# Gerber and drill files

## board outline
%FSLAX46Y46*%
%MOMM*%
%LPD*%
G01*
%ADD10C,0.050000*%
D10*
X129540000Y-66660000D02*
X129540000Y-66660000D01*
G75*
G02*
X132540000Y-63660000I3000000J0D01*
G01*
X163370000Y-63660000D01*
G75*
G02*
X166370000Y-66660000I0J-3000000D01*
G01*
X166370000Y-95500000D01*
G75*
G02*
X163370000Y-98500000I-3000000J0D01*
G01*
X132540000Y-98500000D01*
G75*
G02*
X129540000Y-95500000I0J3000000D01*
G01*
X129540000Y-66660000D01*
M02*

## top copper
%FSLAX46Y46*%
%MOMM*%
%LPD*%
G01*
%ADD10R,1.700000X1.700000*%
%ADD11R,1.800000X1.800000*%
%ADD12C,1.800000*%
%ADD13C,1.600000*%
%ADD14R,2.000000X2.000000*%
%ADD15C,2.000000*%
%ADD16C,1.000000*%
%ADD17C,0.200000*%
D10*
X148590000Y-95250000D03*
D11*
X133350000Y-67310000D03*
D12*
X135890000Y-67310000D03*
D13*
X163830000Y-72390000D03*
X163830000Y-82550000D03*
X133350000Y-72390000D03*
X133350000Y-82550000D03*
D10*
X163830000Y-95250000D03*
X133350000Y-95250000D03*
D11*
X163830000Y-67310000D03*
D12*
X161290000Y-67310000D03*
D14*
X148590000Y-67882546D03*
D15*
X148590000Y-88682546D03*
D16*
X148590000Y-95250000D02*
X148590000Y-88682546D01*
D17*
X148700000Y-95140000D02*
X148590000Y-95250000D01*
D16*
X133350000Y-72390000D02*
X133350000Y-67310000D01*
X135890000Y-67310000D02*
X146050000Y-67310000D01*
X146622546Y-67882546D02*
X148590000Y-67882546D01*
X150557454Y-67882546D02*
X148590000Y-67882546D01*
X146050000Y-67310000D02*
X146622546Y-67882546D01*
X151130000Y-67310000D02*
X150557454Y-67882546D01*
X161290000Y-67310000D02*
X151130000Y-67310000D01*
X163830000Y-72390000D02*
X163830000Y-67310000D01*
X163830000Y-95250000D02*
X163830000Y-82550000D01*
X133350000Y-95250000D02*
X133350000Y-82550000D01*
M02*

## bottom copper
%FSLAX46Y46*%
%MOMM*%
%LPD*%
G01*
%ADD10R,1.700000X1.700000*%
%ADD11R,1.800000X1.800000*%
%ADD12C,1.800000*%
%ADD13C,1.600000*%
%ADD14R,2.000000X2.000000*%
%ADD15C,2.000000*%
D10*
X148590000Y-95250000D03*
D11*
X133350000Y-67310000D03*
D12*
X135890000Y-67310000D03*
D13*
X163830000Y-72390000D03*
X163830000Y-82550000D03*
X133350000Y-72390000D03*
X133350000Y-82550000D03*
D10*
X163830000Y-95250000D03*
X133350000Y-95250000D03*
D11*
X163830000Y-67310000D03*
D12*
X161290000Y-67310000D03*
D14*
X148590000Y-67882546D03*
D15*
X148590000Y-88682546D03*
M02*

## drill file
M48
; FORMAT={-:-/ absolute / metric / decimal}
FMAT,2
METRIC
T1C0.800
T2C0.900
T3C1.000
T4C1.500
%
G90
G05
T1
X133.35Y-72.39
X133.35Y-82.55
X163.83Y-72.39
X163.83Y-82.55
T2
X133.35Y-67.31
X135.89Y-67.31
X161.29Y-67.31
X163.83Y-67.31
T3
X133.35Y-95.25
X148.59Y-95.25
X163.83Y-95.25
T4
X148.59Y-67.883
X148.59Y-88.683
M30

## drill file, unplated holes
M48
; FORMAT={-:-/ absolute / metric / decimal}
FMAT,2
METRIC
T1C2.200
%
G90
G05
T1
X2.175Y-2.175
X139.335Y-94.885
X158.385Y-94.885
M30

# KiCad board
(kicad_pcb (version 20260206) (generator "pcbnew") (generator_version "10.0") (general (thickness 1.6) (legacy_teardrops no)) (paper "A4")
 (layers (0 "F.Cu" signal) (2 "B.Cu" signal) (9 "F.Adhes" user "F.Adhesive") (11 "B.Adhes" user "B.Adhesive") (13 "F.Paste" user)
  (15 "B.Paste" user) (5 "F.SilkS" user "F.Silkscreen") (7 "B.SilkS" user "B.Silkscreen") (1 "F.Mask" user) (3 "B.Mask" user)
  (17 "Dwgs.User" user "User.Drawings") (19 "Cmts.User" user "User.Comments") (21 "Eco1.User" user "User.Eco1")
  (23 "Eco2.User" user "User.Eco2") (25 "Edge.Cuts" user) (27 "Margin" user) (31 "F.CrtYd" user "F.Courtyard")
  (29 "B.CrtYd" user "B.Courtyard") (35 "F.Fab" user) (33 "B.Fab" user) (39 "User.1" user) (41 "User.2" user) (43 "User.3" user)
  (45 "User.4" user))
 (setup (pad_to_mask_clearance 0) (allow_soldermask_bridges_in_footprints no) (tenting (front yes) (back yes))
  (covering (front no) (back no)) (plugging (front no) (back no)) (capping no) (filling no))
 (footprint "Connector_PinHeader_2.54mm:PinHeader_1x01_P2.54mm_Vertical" (layer "F.Cu") (at 148.59 95.25)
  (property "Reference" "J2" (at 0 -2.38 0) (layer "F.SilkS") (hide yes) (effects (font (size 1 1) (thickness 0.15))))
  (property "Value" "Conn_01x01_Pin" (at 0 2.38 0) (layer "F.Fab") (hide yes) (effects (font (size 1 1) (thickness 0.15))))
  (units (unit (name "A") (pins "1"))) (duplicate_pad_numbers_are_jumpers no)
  (pad "1" thru_hole rect (at 0 0) (size 1.7 1.7) (drill 1) (layers "*.Cu" "*.Mask") (remove_unused_layers no) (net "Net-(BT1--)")))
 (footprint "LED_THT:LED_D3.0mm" (layer "F.Cu") (at 133.35 67.31)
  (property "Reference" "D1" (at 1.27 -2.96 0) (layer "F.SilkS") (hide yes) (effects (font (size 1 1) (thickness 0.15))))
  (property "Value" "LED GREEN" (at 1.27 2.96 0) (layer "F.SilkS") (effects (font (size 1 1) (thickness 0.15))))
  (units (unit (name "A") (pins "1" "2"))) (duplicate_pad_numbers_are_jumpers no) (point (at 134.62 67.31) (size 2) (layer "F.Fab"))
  (pad "1" thru_hole rect (at 0 0) (size 1.8 1.8) (drill 0.9) (layers "*.Cu" "*.Mask") (remove_unused_layers no) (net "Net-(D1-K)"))
  (pad "2" thru_hole circle (at 2.54 0) (size 1.8 1.8) (drill 0.9) (layers "*.Cu" "*.Mask") (remove_unused_layers no) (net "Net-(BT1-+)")))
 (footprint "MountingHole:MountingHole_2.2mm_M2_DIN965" (layer "F.Cu") (at 2.175 2.175)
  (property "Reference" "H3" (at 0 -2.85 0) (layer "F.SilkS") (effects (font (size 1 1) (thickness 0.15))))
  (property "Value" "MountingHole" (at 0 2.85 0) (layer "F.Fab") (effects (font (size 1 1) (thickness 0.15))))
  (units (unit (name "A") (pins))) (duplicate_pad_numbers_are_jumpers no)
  (pad "" np_thru_hole circle (at 0 0) (size 2.2 2.2) (drill 2.2) (layers "*.Cu" "*.Mask")))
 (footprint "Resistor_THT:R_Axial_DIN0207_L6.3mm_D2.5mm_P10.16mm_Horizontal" (layer "F.Cu") (at 163.83 72.39 -90)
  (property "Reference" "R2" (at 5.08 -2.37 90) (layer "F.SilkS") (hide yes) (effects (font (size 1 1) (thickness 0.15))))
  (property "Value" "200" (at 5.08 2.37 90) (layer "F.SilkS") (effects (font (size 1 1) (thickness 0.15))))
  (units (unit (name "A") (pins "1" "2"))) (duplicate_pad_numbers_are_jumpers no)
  (pad "1" thru_hole circle (at 0 0 270) (size 1.6 1.6) (drill 0.8) (layers "*.Cu" "*.Mask") (remove_unused_layers no) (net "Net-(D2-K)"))
  (pad "2" thru_hole circle (at 10.16 0 270) (size 1.6 1.6) (drill 0.8) (layers "*.Cu" "*.Mask") (remove_unused_layers no)
   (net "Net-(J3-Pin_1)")))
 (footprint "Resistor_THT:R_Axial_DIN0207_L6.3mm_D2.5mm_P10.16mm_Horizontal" (layer "F.Cu") (at 133.35 72.39 -90)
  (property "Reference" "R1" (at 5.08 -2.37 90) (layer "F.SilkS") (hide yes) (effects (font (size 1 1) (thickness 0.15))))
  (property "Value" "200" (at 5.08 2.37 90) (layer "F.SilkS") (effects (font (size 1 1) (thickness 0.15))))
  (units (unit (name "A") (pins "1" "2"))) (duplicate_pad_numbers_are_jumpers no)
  (pad "1" thru_hole circle (at 0 0 270) (size 1.6 1.6) (drill 0.8) (layers "*.Cu" "*.Mask") (remove_unused_layers no) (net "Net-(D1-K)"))
  (pad "2" thru_hole circle (at 10.16 0 270) (size 1.6 1.6) (drill 0.8) (layers "*.Cu" "*.Mask") (remove_unused_layers no)
   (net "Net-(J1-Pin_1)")))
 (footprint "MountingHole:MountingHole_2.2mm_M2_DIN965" (layer "F.Cu") (at 139.335 94.885)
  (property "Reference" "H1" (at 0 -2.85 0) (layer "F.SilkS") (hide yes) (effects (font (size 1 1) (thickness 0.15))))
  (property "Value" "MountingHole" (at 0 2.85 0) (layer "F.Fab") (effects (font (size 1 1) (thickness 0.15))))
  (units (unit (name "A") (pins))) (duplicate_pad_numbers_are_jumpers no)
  (pad "" np_thru_hole circle (at 0 0) (size 2.2 2.2) (drill 2.2) (layers "*.Cu" "*.Mask")))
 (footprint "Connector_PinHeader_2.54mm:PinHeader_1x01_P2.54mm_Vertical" (layer "F.Cu") (at 163.83 95.25)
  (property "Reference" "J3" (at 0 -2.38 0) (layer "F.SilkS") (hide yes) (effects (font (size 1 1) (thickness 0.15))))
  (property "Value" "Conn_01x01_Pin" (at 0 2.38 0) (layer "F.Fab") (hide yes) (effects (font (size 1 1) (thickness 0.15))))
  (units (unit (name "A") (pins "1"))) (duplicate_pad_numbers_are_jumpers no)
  (pad "1" thru_hole rect (at 0 0) (size 1.7 1.7) (drill 1) (layers "*.Cu" "*.Mask") (remove_unused_layers no) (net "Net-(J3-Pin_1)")))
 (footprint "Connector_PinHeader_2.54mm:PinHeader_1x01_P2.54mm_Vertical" (layer "F.Cu") (at 133.35 95.25)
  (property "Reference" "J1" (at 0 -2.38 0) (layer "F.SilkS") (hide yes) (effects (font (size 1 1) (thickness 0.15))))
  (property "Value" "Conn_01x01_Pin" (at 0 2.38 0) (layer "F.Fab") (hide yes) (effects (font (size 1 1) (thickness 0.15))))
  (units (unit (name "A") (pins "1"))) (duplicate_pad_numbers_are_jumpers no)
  (pad "1" thru_hole rect (at 0 0) (size 1.7 1.7) (drill 1) (layers "*.Cu" "*.Mask") (remove_unused_layers no) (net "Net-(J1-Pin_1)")))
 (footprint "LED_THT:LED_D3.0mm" (layer "F.Cu") (at 163.83 67.31 180)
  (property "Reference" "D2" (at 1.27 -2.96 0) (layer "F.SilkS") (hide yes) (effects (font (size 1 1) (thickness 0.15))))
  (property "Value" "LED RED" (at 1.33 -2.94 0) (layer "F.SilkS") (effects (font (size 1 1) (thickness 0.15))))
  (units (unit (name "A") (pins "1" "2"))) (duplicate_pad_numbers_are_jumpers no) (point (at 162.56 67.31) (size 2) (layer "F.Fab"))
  (pad "1" thru_hole rect (at 0 0 180) (size 1.8 1.8) (drill 0.9) (layers "*.Cu" "*.Mask") (remove_unused_layers no) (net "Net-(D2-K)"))
  (pad "2" thru_hole circle (at 2.54 0 180) (size 1.8 1.8) (drill 0.9) (layers "*.Cu" "*.Mask") (remove_unused_layers no)
   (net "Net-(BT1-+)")))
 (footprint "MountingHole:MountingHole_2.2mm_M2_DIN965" (layer "F.Cu") (at 158.385 94.885)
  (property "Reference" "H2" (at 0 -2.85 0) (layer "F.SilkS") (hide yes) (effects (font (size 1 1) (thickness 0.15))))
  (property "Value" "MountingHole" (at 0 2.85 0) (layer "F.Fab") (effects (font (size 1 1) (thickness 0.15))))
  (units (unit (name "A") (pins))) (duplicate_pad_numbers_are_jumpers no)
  (pad "" np_thru_hole circle (at 0 0) (size 2.2 2.2) (drill 2.2) (layers "*.Cu" "*.Mask")))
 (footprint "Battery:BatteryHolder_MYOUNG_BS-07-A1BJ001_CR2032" (layer "F.Cu") (at 148.59 67.882546 -90)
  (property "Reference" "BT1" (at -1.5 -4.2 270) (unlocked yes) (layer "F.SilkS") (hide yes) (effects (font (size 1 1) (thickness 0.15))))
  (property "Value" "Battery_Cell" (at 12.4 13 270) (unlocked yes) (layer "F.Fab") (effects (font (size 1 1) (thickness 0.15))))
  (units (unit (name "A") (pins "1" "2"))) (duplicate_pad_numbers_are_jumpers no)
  (pad "1" thru_hole rect (at 0 0 90) (size 2 2) (drill 1.5) (layers "*.Cu" "*.Mask") (remove_unused_layers no) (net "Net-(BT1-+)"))
  (pad "2" thru_hole circle (at 20.8 0 90) (size 2 2) (drill 1.5) (layers "*.Cu" "*.Mask") (remove_unused_layers no) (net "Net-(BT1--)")))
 (gr_rect (start 129.54 63.66) (end 166.37 98.5) (radius 3) (stroke (width 0.05) (type solid)) (fill no) (layer "Edge.Cuts"))
 (segment (start 148.59 95.25) (end 148.59 88.682546) (width 1) (layer "F.Cu") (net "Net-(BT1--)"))
 (segment (start 148.7 95.14) (end 148.59 95.25) (width 0.2) (layer "F.Cu") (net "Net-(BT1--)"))
 (segment (start 133.35 72.39) (end 133.35 67.31) (width 1) (layer "F.Cu") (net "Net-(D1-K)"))
 (segment (start 135.89 67.31) (end 146.05 67.31) (width 1) (layer "F.Cu") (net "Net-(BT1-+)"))
 (segment (start 146.622546 67.882546) (end 148.59 67.882546) (width 1) (layer "F.Cu") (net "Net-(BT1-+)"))
 (segment (start 150.557454 67.882546) (end 148.59 67.882546) (width 1) (layer "F.Cu") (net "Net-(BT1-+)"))
 (segment (start 146.05 67.31) (end 146.622546 67.882546) (width 1) (layer "F.Cu") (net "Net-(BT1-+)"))
 (segment (start 151.13 67.31) (end 150.557454 67.882546) (width 1) (layer "F.Cu") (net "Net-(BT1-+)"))
 (segment (start 161.29 67.31) (end 151.13 67.31) (width 1) (layer "F.Cu") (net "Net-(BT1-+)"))
 (segment (start 163.83 72.39) (end 163.83 67.31) (width 1) (layer "F.Cu") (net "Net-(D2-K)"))
 (segment (start 163.83 95.25) (end 163.83 82.55) (width 1) (layer "F.Cu") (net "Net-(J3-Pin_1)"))
 (segment (start 133.35 95.25) (end 133.35 82.55) (width 1) (layer "F.Cu") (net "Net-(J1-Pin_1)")))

